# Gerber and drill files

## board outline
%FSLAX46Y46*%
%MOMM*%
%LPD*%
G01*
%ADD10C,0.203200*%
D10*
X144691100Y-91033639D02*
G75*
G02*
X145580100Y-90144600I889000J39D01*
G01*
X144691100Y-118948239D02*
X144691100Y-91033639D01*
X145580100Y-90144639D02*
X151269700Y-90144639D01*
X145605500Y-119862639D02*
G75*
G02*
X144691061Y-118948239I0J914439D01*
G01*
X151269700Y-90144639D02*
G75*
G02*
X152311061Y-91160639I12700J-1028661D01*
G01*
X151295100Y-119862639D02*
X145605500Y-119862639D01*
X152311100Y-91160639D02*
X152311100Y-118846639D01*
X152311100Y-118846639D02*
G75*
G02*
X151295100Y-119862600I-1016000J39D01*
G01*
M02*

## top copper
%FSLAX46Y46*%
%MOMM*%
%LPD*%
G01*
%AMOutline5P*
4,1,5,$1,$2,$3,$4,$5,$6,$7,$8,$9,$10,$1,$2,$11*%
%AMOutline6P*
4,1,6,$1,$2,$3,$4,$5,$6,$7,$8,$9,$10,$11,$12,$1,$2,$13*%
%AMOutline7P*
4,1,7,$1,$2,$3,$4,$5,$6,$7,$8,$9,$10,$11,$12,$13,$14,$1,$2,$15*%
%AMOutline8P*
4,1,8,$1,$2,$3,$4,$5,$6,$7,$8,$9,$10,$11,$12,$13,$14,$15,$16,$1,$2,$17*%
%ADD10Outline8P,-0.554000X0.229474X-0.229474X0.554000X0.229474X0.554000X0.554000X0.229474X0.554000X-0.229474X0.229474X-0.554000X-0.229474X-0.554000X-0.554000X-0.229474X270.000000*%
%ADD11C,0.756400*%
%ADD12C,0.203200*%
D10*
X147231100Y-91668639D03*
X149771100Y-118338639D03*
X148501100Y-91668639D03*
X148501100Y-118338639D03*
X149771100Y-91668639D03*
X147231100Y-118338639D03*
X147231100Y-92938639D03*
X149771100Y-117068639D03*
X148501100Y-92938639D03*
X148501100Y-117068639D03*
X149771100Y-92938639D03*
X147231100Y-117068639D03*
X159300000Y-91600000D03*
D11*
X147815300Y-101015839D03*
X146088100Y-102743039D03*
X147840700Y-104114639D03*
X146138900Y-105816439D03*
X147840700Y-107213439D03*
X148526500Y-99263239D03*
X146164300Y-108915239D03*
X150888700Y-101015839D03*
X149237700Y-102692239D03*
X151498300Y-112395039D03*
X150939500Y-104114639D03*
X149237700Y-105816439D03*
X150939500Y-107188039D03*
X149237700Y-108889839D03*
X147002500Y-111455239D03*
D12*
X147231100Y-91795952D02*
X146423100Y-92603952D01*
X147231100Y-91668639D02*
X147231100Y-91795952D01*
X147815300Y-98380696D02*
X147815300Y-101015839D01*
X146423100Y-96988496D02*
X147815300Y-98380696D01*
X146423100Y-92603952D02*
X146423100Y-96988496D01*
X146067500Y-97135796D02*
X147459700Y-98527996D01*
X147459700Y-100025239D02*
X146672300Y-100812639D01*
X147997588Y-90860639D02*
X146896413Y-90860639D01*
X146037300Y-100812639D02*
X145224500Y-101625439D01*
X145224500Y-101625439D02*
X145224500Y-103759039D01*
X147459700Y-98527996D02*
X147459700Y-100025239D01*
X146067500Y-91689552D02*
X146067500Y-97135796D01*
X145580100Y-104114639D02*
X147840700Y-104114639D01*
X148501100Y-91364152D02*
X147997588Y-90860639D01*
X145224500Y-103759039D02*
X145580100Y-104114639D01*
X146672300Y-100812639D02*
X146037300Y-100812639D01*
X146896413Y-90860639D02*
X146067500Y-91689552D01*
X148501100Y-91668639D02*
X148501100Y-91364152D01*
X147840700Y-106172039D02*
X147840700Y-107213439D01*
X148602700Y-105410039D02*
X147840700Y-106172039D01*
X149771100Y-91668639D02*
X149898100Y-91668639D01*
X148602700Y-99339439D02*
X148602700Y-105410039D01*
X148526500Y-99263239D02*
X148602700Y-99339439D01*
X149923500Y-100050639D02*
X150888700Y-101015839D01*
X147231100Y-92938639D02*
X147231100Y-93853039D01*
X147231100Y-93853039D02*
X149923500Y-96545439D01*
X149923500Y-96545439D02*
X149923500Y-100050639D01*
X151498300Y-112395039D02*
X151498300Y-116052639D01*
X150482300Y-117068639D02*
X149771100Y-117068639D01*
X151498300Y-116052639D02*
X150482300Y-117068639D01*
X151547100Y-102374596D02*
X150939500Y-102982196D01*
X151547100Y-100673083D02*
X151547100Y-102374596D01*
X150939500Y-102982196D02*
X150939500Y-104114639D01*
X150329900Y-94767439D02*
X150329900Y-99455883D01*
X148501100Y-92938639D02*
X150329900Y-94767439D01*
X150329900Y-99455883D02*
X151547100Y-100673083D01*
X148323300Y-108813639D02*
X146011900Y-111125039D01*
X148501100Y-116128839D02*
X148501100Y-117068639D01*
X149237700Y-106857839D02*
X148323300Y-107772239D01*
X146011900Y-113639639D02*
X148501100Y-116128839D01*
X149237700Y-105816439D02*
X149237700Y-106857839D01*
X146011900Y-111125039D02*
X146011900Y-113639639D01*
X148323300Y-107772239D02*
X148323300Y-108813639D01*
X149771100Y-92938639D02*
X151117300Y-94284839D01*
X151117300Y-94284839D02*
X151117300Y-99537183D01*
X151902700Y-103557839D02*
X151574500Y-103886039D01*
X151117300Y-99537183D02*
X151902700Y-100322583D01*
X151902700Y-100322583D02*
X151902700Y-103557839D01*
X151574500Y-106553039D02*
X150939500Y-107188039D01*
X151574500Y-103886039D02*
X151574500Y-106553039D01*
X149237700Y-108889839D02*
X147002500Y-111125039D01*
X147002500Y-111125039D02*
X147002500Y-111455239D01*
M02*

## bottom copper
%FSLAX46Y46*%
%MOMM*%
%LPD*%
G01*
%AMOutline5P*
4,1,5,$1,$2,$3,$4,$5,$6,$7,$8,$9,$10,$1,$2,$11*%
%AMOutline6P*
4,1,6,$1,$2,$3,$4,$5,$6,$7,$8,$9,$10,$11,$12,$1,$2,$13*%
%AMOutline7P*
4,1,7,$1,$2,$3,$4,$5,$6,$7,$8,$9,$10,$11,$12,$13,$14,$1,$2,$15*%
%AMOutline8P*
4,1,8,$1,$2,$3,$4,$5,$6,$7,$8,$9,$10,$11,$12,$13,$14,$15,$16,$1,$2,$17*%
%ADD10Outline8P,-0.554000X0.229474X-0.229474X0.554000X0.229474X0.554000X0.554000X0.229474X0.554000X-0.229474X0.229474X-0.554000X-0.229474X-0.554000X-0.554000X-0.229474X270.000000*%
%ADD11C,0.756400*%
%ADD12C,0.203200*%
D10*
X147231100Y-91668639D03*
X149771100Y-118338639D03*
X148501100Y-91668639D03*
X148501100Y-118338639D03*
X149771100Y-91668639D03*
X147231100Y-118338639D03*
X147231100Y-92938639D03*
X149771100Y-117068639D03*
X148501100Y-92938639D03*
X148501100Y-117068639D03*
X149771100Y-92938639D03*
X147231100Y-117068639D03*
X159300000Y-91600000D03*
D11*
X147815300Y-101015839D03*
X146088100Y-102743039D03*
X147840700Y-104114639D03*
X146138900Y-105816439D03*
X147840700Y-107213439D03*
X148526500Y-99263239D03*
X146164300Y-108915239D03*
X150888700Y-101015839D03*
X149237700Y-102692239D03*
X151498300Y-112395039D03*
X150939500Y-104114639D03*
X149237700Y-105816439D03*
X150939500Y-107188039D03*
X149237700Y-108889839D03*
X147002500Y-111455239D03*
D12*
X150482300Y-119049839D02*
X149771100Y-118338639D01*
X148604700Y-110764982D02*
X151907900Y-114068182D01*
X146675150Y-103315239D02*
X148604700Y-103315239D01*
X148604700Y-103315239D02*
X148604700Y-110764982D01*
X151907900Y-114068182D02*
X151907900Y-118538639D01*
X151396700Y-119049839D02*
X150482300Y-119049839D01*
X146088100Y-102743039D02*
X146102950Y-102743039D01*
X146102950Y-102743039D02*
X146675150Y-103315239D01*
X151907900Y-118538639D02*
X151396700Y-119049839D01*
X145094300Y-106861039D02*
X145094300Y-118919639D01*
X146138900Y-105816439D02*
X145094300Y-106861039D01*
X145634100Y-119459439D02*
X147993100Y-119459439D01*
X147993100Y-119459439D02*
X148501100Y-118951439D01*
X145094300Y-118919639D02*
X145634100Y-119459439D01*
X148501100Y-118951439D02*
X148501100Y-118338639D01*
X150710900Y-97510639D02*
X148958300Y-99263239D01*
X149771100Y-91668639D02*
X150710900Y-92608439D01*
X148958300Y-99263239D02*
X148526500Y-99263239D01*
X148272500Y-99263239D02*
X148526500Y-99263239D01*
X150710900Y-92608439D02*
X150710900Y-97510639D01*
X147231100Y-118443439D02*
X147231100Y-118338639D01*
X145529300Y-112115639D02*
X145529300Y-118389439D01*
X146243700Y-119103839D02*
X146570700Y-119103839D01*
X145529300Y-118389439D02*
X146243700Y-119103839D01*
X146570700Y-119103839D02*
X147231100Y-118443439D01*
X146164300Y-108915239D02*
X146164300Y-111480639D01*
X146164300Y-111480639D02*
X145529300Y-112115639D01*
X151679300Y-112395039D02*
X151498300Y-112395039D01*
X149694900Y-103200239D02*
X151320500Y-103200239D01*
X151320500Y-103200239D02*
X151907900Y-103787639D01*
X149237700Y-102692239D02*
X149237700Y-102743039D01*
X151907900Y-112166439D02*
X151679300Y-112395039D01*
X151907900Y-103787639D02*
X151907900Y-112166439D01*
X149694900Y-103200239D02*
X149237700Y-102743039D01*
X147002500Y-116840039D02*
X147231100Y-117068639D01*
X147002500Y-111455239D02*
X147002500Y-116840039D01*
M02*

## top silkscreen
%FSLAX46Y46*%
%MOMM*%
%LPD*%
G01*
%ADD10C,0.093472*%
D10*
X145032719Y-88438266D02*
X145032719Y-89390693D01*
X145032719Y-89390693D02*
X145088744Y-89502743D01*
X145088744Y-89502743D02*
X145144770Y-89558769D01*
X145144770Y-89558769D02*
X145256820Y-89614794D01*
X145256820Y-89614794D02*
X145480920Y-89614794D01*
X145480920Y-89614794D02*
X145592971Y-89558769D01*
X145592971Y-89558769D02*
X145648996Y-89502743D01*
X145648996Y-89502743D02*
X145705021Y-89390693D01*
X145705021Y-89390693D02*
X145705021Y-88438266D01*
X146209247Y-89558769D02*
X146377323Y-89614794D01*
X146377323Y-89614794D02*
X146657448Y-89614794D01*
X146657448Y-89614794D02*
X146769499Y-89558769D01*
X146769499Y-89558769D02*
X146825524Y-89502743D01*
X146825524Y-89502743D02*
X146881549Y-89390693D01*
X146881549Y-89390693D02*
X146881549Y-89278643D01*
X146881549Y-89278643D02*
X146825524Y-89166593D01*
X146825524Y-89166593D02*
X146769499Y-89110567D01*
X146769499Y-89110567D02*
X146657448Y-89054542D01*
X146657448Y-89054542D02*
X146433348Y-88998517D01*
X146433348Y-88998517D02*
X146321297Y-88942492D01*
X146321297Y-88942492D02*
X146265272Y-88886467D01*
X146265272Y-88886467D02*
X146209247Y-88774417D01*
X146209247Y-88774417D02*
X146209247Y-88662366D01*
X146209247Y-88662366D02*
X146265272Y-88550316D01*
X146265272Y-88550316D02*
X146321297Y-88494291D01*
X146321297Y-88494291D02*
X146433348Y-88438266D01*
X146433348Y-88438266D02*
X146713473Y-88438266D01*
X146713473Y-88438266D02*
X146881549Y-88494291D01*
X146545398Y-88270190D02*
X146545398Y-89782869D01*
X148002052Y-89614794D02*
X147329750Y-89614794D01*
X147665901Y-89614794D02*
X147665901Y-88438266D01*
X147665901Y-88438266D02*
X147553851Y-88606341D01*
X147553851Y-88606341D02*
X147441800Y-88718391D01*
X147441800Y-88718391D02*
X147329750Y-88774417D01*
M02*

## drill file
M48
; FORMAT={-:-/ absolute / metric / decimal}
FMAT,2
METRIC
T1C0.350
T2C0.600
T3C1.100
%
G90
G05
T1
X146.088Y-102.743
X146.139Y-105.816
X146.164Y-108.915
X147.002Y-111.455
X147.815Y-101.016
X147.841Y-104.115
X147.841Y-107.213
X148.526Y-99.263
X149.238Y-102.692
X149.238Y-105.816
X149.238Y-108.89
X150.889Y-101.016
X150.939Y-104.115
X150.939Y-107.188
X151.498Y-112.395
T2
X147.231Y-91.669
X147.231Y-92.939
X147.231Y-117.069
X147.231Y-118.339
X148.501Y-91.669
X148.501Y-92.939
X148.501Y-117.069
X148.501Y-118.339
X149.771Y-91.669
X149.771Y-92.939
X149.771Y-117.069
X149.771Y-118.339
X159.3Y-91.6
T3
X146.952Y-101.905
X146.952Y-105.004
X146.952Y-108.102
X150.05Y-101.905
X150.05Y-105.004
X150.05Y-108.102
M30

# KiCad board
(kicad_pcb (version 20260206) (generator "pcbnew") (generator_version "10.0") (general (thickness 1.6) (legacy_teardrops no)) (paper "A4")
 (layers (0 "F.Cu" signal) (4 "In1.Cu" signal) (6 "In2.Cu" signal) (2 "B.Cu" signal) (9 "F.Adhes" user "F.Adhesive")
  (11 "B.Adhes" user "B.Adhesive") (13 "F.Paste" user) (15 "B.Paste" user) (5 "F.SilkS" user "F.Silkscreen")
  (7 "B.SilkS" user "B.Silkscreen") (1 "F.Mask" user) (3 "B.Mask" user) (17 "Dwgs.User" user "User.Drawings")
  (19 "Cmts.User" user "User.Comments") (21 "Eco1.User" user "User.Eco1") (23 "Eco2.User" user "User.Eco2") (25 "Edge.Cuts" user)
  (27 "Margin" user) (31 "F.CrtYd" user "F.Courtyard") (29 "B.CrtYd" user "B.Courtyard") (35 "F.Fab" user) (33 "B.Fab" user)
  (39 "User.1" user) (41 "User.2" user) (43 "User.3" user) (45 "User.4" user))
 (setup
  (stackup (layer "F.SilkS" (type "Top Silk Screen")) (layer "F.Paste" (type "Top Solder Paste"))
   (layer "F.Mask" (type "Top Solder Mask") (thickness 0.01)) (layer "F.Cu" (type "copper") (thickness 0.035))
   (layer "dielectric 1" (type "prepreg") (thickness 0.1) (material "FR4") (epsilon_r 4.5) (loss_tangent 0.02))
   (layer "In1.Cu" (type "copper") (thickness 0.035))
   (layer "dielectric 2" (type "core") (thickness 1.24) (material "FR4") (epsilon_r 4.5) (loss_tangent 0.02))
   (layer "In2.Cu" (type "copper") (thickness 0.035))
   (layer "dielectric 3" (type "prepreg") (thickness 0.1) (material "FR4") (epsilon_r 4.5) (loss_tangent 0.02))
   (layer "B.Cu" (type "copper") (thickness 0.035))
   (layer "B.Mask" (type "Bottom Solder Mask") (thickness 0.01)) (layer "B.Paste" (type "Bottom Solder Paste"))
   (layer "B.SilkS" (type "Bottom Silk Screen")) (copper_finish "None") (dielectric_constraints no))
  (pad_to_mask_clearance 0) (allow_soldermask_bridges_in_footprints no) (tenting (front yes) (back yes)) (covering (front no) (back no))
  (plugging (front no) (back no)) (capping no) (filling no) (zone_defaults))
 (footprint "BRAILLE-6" (layer "F.Cu") (at 148.5011 105.003639)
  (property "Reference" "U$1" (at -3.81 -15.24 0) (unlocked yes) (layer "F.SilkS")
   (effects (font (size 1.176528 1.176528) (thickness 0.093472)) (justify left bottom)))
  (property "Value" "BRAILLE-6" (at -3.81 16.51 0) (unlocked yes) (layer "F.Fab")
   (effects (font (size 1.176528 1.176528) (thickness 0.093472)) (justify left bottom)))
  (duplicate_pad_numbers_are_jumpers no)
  (pad "P$1" thru_hole roundrect (at -1.27 -13.335 270) (size 1.108 1.108) (drill 0.6) (layers "*.Cu" "*.Mask") (remove_unused_layers no)
   (roundrect_rratio 0.25) (chamfer_ratio 0.2928932188) (chamfer top_left top_right bottom_left bottom_right) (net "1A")
   (solder_mask_margin 0.1016) (thermal_bridge_angle 0))
  (pad "P$2" thru_hole roundrect (at 1.27 13.335 270) (size 1.108 1.108) (drill 0.6) (layers "*.Cu" "*.Mask") (remove_unused_layers no)
   (roundrect_rratio 0.25) (chamfer_ratio 0.2928932188) (chamfer top_left top_right bottom_left bottom_right) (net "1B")
   (solder_mask_margin 0.1016) (thermal_bridge_angle 0))
  (pad "P$3" thru_hole roundrect (at 0 -13.335 270) (size 1.108 1.108) (drill 0.6) (layers "*.Cu" "*.Mask") (remove_unused_layers no)
   (roundrect_rratio 0.25) (chamfer_ratio 0.2928932188) (chamfer top_left top_right bottom_left bottom_right) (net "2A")
   (solder_mask_margin 0.1016) (thermal_bridge_angle 0))
  (pad "P$4" thru_hole roundrect (at 0 13.335 270) (size 1.108 1.108) (drill 0.6) (layers "*.Cu" "*.Mask") (remove_unused_layers no)
   (roundrect_rratio 0.25) (chamfer_ratio 0.2928932188) (chamfer top_left top_right bottom_left bottom_right) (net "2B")
   (solder_mask_margin 0.1016) (thermal_bridge_angle 0))
  (pad "P$5" thru_hole roundrect (at 1.27 -13.335 270) (size 1.108 1.108) (drill 0.6) (layers "*.Cu" "*.Mask") (remove_unused_layers no)
   (roundrect_rratio 0.25) (chamfer_ratio 0.2928932188) (chamfer top_left top_right bottom_left bottom_right) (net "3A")
   (solder_mask_margin 0.1016) (thermal_bridge_angle 0))
  (pad "P$6" thru_hole roundrect (at -1.27 13.335 270) (size 1.108 1.108) (drill 0.6) (layers "*.Cu" "*.Mask") (remove_unused_layers no)
   (roundrect_rratio 0.25) (chamfer_ratio 0.2928932188) (chamfer top_left top_right bottom_left bottom_right) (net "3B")
   (solder_mask_margin 0.1016) (thermal_bridge_angle 0))
  (pad "P$7" thru_hole roundrect (at -1.27 -12.065 270) (size 1.108 1.108) (drill 0.6) (layers "*.Cu" "*.Mask") (remove_unused_layers no)
   (roundrect_rratio 0.25) (chamfer_ratio 0.2928932188) (chamfer top_left top_right bottom_left bottom_right) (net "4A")
   (solder_mask_margin 0.1016) (thermal_bridge_angle 0))
  (pad "P$8" thru_hole roundrect (at 1.27 12.065 270) (size 1.108 1.108) (drill 0.6) (layers "*.Cu" "*.Mask") (remove_unused_layers no)
   (roundrect_rratio 0.25) (chamfer_ratio 0.2928932188) (chamfer top_left top_right bottom_left bottom_right) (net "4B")
   (solder_mask_margin 0.1016) (thermal_bridge_angle 0))
  (pad "P$9" thru_hole roundrect (at 0 -12.065 270) (size 1.108 1.108) (drill 0.6) (layers "*.Cu" "*.Mask") (remove_unused_layers no)
   (roundrect_rratio 0.25) (chamfer_ratio 0.2928932188) (chamfer top_left top_right bottom_left bottom_right) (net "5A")
   (solder_mask_margin 0.1016) (thermal_bridge_angle 0))
  (pad "P$10" thru_hole roundrect (at 0 12.065 270) (size 1.108 1.108) (drill 0.6) (layers "*.Cu" "*.Mask") (remove_unused_layers no)
   (roundrect_rratio 0.25) (chamfer_ratio 0.2928932188) (chamfer top_left top_right bottom_left bottom_right) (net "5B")
   (solder_mask_margin 0.1016) (thermal_bridge_angle 0))
  (pad "P$11" thru_hole roundrect (at 1.27 -12.065 270) (size 1.108 1.108) (drill 0.6) (layers "*.Cu" "*.Mask") (remove_unused_layers no)
   (roundrect_rratio 0.25) (chamfer_ratio 0.2928932188) (chamfer top_left top_right bottom_left bottom_right) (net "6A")
   (solder_mask_margin 0.1016) (thermal_bridge_angle 0))
  (pad "P$12" thru_hole roundrect (at -1.27 12.065 270) (size 1.108 1.108) (drill 0.6) (layers "*.Cu" "*.Mask") (remove_unused_layers no)
   (roundrect_rratio 0.25) (chamfer_ratio 0.2928932188) (chamfer top_left top_right bottom_left bottom_right) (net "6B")
   (solder_mask_margin 0.1016) (thermal_bridge_angle 0)))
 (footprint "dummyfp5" (layer "F.Cu") (at 150.0505 108.102439)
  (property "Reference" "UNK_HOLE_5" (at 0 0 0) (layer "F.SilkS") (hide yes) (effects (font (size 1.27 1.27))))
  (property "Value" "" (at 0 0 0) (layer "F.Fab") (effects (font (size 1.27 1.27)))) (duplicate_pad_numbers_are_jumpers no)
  (pad "" np_thru_hole circle (at 0 0) (size 1.1 1.1) (drill 1.1) (layers "*.Cu" "*.Mask")))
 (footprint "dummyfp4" (layer "F.Cu") (at 146.9517 108.102439)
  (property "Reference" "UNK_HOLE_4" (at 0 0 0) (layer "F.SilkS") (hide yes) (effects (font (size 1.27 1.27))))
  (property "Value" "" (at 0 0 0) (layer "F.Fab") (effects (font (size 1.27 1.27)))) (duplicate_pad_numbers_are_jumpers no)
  (pad "" np_thru_hole circle (at 0 0) (size 1.1 1.1) (drill 1.1) (layers "*.Cu" "*.Mask")))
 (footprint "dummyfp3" (layer "F.Cu") (at 150.0505 105.003639)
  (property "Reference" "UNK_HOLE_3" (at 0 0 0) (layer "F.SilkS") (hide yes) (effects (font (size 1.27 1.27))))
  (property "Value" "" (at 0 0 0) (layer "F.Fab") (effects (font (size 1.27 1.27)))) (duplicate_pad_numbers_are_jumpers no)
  (pad "" np_thru_hole circle (at 0 0) (size 1.1 1.1) (drill 1.1) (layers "*.Cu" "*.Mask")))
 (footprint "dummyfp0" (layer "F.Cu") (at 146.9517 101.904839)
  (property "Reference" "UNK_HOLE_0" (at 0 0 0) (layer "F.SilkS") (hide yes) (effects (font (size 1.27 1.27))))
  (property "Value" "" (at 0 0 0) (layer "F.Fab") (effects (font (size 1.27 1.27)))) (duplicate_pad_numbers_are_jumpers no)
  (pad "" np_thru_hole circle (at 0 0) (size 1.1 1.1) (drill 1.1) (layers "*.Cu" "*.Mask")))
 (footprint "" (layer "F.Cu") (at 159.3 91.6)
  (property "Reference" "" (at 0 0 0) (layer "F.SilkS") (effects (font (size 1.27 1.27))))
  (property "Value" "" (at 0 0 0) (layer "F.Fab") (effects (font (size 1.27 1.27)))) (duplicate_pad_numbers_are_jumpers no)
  (pad "P$1" thru_hole roundrect (at 0 0 270) (size 1.108 1.108) (drill 0.6) (layers "*.Cu" "*.Mask") (remove_unused_layers no)
   (roundrect_rratio 0.25) (chamfer_ratio 0.2928932188) (chamfer top_left top_right bottom_left bottom_right) (solder_mask_margin 0.1016)
   (thermal_bridge_angle 0)))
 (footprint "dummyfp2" (layer "F.Cu") (at 146.9517 105.003639)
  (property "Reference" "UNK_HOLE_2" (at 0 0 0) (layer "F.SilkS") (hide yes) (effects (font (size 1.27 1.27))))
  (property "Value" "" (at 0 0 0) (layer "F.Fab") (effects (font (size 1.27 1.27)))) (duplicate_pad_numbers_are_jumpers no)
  (pad "" np_thru_hole circle (at 0 0) (size 1.1 1.1) (drill 1.1) (layers "*.Cu" "*.Mask")))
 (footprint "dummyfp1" (layer "F.Cu") (at 150.0505 101.904839)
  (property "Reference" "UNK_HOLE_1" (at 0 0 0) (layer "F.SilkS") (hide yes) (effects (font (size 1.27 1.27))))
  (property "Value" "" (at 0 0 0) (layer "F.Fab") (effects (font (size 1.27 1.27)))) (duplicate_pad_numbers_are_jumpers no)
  (pad "" np_thru_hole circle (at 0 0) (size 1.1 1.1) (drill 1.1) (layers "*.Cu" "*.Mask")))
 (gr_arc (start 144.6911 91.033639) (mid 144.951482 90.405021) (end 145.5801 90.144639) (stroke (width 0.2032) (type solid))
  (layer "Edge.Cuts"))
 (gr_line (start 144.6911 118.948239) (end 144.6911 91.033639) (stroke (width 0.2032) (type solid)) (layer "Edge.Cuts"))
 (gr_line (start 145.5801 90.144639) (end 151.2697 90.144639) (stroke (width 0.2032) (type solid)) (layer "Edge.Cuts"))
 (gr_arc (start 145.6055 119.862639) (mid 144.958922 119.594817) (end 144.6911 118.948239) (stroke (width 0.2032) (type solid))
  (layer "Edge.Cuts"))
 (gr_arc (start 151.2697 90.144639) (mid 152.00082 90.436958) (end 152.3111 91.160639) (stroke (width 0.2032) (type solid))
  (layer "Edge.Cuts"))
 (gr_line (start 151.2951 119.862639) (end 145.6055 119.862639) (stroke (width 0.2032) (type solid)) (layer "Edge.Cuts"))
 (gr_line (start 152.3111 91.160639) (end 152.3111 118.846639) (stroke (width 0.2032) (type solid)) (layer "Edge.Cuts"))
 (gr_arc (start 152.3111 118.846639) (mid 152.01352 119.565059) (end 151.2951 119.862639) (stroke (width 0.2032) (type solid))
  (layer "Edge.Cuts"))
 (segment (start 147.2311 91.795952) (end 146.4231 92.603952) (width 0.2032) (layer "F.Cu") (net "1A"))
 (segment (start 147.2311 91.668639) (end 147.2311 91.795952) (width 0.2032) (layer "F.Cu") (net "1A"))
 (segment (start 147.8153 98.380696) (end 147.8153 101.015839) (width 0.2032) (layer "F.Cu") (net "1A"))
 (segment (start 146.4231 96.988496) (end 147.8153 98.380696) (width 0.2032) (layer "F.Cu") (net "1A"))
 (segment (start 146.4231 92.603952) (end 146.4231 96.988496) (width 0.2032) (layer "F.Cu") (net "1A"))
 (via (at 147.8153 101.015839) (size 0.7564) (drill 0.35) (layers "F.Cu" "B.Cu") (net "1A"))
 (via (at 146.0881 102.743039) (size 0.7564) (drill 0.35) (layers "F.Cu" "B.Cu") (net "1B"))
 (segment (start 150.4823 119.049839) (end 149.7711 118.338639) (width 0.2032) (layer "B.Cu") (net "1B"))
 (segment (start 148.6047 110.764982) (end 151.9079 114.068182) (width 0.2032) (layer "B.Cu") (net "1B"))
 (segment (start 146.67515 103.315239) (end 148.6047 103.315239) (width 0.2032) (layer "B.Cu") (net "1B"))
 (segment (start 148.6047 103.315239) (end 148.6047 110.764982) (width 0.2032) (layer "B.Cu") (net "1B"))
 (segment (start 151.9079 114.068182) (end 151.9079 118.538639) (width 0.2032) (layer "B.Cu") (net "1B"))
 (segment (start 151.3967 119.049839) (end 150.4823 119.049839) (width 0.2032) (layer "B.Cu") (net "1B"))
 (segment (start 146.0881 102.743039) (end 146.10295 102.743039) (width 0.2032) (layer "B.Cu") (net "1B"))
 (segment (start 146.10295 102.743039) (end 146.67515 103.315239) (width 0.2032) (layer "B.Cu") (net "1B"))
 (segment (start 151.9079 118.538639) (end 151.3967 119.049839) (width 0.2032) (layer "B.Cu") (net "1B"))
 (segment (start 146.0675 97.135796) (end 147.4597 98.527996) (width 0.2032) (layer "F.Cu") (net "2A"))
 (segment (start 147.4597 100.025239) (end 146.6723 100.812639) (width 0.2032) (layer "F.Cu") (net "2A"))
 (segment (start 147.997588 90.860639) (end 146.896413 90.860639) (width 0.2032) (layer "F.Cu") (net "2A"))
 (segment (start 146.0373 100.812639) (end 145.2245 101.625439) (width 0.2032) (layer "F.Cu") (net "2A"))
 (segment (start 145.2245 101.625439) (end 145.2245 103.759039) (width 0.2032) (layer "F.Cu") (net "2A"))
 (segment (start 147.4597 98.527996) (end 147.4597 100.025239) (width 0.2032) (layer "F.Cu") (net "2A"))
 (segment (start 146.0675 91.689552) (end 146.0675 97.135796) (width 0.2032) (layer "F.Cu") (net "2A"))
 (segment (start 145.5801 104.114639) (end 147.8407 104.114639) (width 0.2032) (layer "F.Cu") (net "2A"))
 (segment (start 148.5011 91.364152) (end 147.997588 90.860639) (width 0.2032) (layer "F.Cu") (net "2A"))
 (segment (start 145.2245 103.759039) (end 145.5801 104.114639) (width 0.2032) (layer "F.Cu") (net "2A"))
 (segment (start 146.6723 100.812639) (end 146.0373 100.812639) (width 0.2032) (layer "F.Cu") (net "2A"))
 (segment (start 146.896413 90.860639) (end 146.0675 91.689552) (width 0.2032) (layer "F.Cu") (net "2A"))
 (segment (start 148.5011 91.668639) (end 148.5011 91.364152) (width 0.2032) (layer "F.Cu") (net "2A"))
 (via (at 147.8407 104.114639) (size 0.7564) (drill 0.35) (layers "F.Cu" "B.Cu") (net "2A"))
 (via (at 146.1389 105.816439) (size 0.7564) (drill 0.35) (layers "F.Cu" "B.Cu") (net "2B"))
 (segment (start 145.0943 106.861039) (end 145.0943 118.919639) (width 0.2032) (layer "B.Cu") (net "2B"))
 (segment (start 146.1389 105.816439) (end 145.0943 106.861039) (width 0.2032) (layer "B.Cu") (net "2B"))
 (segment (start 145.6341 119.459439) (end 147.9931 119.459439) (width 0.2032) (layer "B.Cu") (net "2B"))
 (segment (start 147.9931 119.459439) (end 148.5011 118.951439) (width 0.2032) (layer "B.Cu") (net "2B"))
 (segment (start 145.0943 118.919639) (end 145.6341 119.459439) (width 0.2032) (layer "B.Cu") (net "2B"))
 (segment (start 148.5011 118.951439) (end 148.5011 118.338639) (width 0.2032) (layer "B.Cu") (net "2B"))
 (segment (start 147.8407 106.172039) (end 147.8407 107.213439) (width 0.2032) (layer "F.Cu") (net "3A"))
 (segment (start 148.6027 105.410039) (end 147.8407 106.172039) (width 0.2032) (layer "F.Cu") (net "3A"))
 (segment (start 149.7711 91.668639) (end 149.8981 91.668639) (width 0.2032) (layer "F.Cu") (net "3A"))
 (segment (start 148.6027 99.339439) (end 148.6027 105.410039) (width 0.2032) (layer "F.Cu") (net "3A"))
 (segment (start 148.5265 99.263239) (end 148.6027 99.339439) (width 0.2032) (layer "F.Cu") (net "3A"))
 (via (at 147.8407 107.213439) (size 0.7564) (drill 0.35) (layers "F.Cu" "B.Cu") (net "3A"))
 (via (at 148.5265 99.263239) (size 0.7564) (drill 0.35) (layers "F.Cu" "B.Cu") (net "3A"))
 (segment (start 150.7109 97.510639) (end 148.9583 99.263239) (width 0.2032) (layer "B.Cu") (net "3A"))
 (segment (start 149.7711 91.668639) (end 150.7109 92.608439) (width 0.2032) (layer "B.Cu") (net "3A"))
 (segment (start 148.9583 99.263239) (end 148.5265 99.263239) (width 0.2032) (layer "B.Cu") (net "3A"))
 (segment (start 148.2725 99.263239) (end 148.5265 99.263239) (width 0.2032) (layer "B.Cu") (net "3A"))
 (segment (start 150.7109 92.608439) (end 150.7109 97.510639) (width 0.2032) (layer "B.Cu") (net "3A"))
 (via (at 146.1643 108.915239) (size 0.7564) (drill 0.35) (layers "F.Cu" "B.Cu") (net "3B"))
 (segment (start 147.2311 118.443439) (end 147.2311 118.338639) (width 0.2032) (layer "B.Cu") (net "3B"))
 (segment (start 145.5293 112.115639) (end 145.5293 118.389439) (width 0.2032) (layer "B.Cu") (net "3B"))
 (segment (start 146.2437 119.103839) (end 146.5707 119.103839) (width 0.2032) (layer "B.Cu") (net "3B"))
 (segment (start 145.5293 118.389439) (end 146.2437 119.103839) (width 0.2032) (layer "B.Cu") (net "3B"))
 (segment (start 146.5707 119.103839) (end 147.2311 118.443439) (width 0.2032) (layer "B.Cu") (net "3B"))
 (segment (start 146.1643 108.915239) (end 146.1643 111.480639) (width 0.2032) (layer "B.Cu") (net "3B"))
 (segment (start 146.1643 111.480639) (end 145.5293 112.115639) (width 0.2032) (layer "B.Cu") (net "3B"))
 (segment (start 149.9235 100.050639) (end 150.8887 101.015839) (width 0.2032) (layer "F.Cu") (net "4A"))
 (segment (start 147.2311 92.938639) (end 147.2311 93.853039) (width 0.2032) (layer "F.Cu") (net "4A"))
 (segment (start 147.2311 93.853039) (end 149.9235 96.545439) (width 0.2032) (layer "F.Cu") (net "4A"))
 (segment (start 149.9235 96.545439) (end 149.9235 100.050639) (width 0.2032) (layer "F.Cu") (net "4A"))
 (via (at 150.8887 101.015839) (size 0.7564) (drill 0.35) (layers "F.Cu" "B.Cu") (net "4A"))
 (segment (start 151.4983 112.395039) (end 151.4983 116.052639) (width 0.2032) (layer "F.Cu") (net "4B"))
 (segment (start 150.4823 117.068639) (end 149.7711 117.068639) (width 0.2032) (layer "F.Cu") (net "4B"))
 (segment (start 151.4983 116.052639) (end 150.4823 117.068639) (width 0.2032) (layer "F.Cu") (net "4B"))
 (via (at 149.2377 102.692239) (size 0.7564) (drill 0.35) (layers "F.Cu" "B.Cu") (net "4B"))
 (via (at 151.4983 112.395039) (size 0.7564) (drill 0.35) (layers "F.Cu" "B.Cu") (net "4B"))
 (segment (start 151.6793 112.395039) (end 151.4983 112.395039) (width 0.2032) (layer "B.Cu") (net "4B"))
 (segment (start 149.6949 103.200239) (end 151.3205 103.200239) (width 0.2032) (layer "B.Cu") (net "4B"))
 (segment (start 151.3205 103.200239) (end 151.9079 103.787639) (width 0.2032) (layer "B.Cu") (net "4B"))
 (segment (start 149.2377 102.692239) (end 149.2377 102.743039) (width 0.2032) (layer "B.Cu") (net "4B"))
 (segment (start 151.9079 112.166439) (end 151.6793 112.395039) (width 0.2032) (layer "B.Cu") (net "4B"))
 (segment (start 151.9079 103.787639) (end 151.9079 112.166439) (width 0.2032) (layer "B.Cu") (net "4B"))
 (segment (start 149.6949 103.200239) (end 149.2377 102.743039) (width 0.2032) (layer "B.Cu") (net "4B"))
 (segment (start 151.5471 102.374596) (end 150.9395 102.982196) (width 0.2032) (layer "F.Cu") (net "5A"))
 (segment (start 151.5471 100.673083) (end 151.5471 102.374596) (width 0.2032) (layer "F.Cu") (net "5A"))
 (segment (start 150.9395 102.982196) (end 150.9395 104.114639) (width 0.2032) (layer "F.Cu") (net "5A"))
 (segment (start 150.3299 94.767439) (end 150.3299 99.455883) (width 0.2032) (layer "F.Cu") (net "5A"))
 (segment (start 148.5011 92.938639) (end 150.3299 94.767439) (width 0.2032) (layer "F.Cu") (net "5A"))
 (segment (start 150.3299 99.455883) (end 151.5471 100.673083) (width 0.2032) (layer "F.Cu") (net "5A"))
 (via (at 150.9395 104.114639) (size 0.7564) (drill 0.35) (layers "F.Cu" "B.Cu") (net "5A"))
 (segment (start 148.3233 108.813639) (end 146.0119 111.125039) (width 0.2032) (layer "F.Cu") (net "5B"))
 (segment (start 148.5011 116.128839) (end 148.5011 117.068639) (width 0.2032) (layer "F.Cu") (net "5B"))
 (segment (start 149.2377 106.857839) (end 148.3233 107.772239) (width 0.2032) (layer "F.Cu") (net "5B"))
 (segment (start 146.0119 113.639639) (end 148.5011 116.128839) (width 0.2032) (layer "F.Cu") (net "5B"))
 (segment (start 149.2377 105.816439) (end 149.2377 106.857839) (width 0.2032) (layer "F.Cu") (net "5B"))
 (segment (start 146.0119 111.125039) (end 146.0119 113.639639) (width 0.2032) (layer "F.Cu") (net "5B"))
 (segment (start 148.3233 107.772239) (end 148.3233 108.813639) (width 0.2032) (layer "F.Cu") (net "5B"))
 (via (at 149.2377 105.816439) (size 0.7564) (drill 0.35) (layers "F.Cu" "B.Cu") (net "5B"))
 (segment (start 149.7711 92.938639) (end 151.1173 94.284839) (width 0.2032) (layer "F.Cu") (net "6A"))
 (segment (start 151.1173 94.284839) (end 151.1173 99.537183) (width 0.2032) (layer "F.Cu") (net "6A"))
 (segment (start 151.9027 103.557839) (end 151.5745 103.886039) (width 0.2032) (layer "F.Cu") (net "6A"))
 (segment (start 151.1173 99.537183) (end 151.9027 100.322583) (width 0.2032) (layer "F.Cu") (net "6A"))
 (segment (start 151.9027 100.322583) (end 151.9027 103.557839) (width 0.2032) (layer "F.Cu") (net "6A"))
 (segment (start 151.5745 106.553039) (end 150.9395 107.188039) (width 0.2032) (layer "F.Cu") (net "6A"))
 (segment (start 151.5745 103.886039) (end 151.5745 106.553039) (width 0.2032) (layer "F.Cu") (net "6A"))
 (via (at 150.9395 107.188039) (size 0.7564) (drill 0.35) (layers "F.Cu" "B.Cu") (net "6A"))
 (segment (start 149.2377 108.889839) (end 147.0025 111.125039) (width 0.2032) (layer "F.Cu") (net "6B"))
 (segment (start 147.0025 111.125039) (end 147.0025 111.455239) (width 0.2032) (layer "F.Cu") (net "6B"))
 (via (at 149.2377 108.889839) (size 0.7564) (drill 0.35) (layers "F.Cu" "B.Cu") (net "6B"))
 (via (at 147.0025 111.455239) (size 0.7564) (drill 0.35) (layers "F.Cu" "B.Cu") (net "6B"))
 (segment (start 147.0025 116.840039) (end 147.2311 117.068639) (width 0.2032) (layer "B.Cu") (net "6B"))
 (segment (start 147.0025 111.455239) (end 147.0025 116.840039) (width 0.2032) (layer "B.Cu") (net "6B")))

